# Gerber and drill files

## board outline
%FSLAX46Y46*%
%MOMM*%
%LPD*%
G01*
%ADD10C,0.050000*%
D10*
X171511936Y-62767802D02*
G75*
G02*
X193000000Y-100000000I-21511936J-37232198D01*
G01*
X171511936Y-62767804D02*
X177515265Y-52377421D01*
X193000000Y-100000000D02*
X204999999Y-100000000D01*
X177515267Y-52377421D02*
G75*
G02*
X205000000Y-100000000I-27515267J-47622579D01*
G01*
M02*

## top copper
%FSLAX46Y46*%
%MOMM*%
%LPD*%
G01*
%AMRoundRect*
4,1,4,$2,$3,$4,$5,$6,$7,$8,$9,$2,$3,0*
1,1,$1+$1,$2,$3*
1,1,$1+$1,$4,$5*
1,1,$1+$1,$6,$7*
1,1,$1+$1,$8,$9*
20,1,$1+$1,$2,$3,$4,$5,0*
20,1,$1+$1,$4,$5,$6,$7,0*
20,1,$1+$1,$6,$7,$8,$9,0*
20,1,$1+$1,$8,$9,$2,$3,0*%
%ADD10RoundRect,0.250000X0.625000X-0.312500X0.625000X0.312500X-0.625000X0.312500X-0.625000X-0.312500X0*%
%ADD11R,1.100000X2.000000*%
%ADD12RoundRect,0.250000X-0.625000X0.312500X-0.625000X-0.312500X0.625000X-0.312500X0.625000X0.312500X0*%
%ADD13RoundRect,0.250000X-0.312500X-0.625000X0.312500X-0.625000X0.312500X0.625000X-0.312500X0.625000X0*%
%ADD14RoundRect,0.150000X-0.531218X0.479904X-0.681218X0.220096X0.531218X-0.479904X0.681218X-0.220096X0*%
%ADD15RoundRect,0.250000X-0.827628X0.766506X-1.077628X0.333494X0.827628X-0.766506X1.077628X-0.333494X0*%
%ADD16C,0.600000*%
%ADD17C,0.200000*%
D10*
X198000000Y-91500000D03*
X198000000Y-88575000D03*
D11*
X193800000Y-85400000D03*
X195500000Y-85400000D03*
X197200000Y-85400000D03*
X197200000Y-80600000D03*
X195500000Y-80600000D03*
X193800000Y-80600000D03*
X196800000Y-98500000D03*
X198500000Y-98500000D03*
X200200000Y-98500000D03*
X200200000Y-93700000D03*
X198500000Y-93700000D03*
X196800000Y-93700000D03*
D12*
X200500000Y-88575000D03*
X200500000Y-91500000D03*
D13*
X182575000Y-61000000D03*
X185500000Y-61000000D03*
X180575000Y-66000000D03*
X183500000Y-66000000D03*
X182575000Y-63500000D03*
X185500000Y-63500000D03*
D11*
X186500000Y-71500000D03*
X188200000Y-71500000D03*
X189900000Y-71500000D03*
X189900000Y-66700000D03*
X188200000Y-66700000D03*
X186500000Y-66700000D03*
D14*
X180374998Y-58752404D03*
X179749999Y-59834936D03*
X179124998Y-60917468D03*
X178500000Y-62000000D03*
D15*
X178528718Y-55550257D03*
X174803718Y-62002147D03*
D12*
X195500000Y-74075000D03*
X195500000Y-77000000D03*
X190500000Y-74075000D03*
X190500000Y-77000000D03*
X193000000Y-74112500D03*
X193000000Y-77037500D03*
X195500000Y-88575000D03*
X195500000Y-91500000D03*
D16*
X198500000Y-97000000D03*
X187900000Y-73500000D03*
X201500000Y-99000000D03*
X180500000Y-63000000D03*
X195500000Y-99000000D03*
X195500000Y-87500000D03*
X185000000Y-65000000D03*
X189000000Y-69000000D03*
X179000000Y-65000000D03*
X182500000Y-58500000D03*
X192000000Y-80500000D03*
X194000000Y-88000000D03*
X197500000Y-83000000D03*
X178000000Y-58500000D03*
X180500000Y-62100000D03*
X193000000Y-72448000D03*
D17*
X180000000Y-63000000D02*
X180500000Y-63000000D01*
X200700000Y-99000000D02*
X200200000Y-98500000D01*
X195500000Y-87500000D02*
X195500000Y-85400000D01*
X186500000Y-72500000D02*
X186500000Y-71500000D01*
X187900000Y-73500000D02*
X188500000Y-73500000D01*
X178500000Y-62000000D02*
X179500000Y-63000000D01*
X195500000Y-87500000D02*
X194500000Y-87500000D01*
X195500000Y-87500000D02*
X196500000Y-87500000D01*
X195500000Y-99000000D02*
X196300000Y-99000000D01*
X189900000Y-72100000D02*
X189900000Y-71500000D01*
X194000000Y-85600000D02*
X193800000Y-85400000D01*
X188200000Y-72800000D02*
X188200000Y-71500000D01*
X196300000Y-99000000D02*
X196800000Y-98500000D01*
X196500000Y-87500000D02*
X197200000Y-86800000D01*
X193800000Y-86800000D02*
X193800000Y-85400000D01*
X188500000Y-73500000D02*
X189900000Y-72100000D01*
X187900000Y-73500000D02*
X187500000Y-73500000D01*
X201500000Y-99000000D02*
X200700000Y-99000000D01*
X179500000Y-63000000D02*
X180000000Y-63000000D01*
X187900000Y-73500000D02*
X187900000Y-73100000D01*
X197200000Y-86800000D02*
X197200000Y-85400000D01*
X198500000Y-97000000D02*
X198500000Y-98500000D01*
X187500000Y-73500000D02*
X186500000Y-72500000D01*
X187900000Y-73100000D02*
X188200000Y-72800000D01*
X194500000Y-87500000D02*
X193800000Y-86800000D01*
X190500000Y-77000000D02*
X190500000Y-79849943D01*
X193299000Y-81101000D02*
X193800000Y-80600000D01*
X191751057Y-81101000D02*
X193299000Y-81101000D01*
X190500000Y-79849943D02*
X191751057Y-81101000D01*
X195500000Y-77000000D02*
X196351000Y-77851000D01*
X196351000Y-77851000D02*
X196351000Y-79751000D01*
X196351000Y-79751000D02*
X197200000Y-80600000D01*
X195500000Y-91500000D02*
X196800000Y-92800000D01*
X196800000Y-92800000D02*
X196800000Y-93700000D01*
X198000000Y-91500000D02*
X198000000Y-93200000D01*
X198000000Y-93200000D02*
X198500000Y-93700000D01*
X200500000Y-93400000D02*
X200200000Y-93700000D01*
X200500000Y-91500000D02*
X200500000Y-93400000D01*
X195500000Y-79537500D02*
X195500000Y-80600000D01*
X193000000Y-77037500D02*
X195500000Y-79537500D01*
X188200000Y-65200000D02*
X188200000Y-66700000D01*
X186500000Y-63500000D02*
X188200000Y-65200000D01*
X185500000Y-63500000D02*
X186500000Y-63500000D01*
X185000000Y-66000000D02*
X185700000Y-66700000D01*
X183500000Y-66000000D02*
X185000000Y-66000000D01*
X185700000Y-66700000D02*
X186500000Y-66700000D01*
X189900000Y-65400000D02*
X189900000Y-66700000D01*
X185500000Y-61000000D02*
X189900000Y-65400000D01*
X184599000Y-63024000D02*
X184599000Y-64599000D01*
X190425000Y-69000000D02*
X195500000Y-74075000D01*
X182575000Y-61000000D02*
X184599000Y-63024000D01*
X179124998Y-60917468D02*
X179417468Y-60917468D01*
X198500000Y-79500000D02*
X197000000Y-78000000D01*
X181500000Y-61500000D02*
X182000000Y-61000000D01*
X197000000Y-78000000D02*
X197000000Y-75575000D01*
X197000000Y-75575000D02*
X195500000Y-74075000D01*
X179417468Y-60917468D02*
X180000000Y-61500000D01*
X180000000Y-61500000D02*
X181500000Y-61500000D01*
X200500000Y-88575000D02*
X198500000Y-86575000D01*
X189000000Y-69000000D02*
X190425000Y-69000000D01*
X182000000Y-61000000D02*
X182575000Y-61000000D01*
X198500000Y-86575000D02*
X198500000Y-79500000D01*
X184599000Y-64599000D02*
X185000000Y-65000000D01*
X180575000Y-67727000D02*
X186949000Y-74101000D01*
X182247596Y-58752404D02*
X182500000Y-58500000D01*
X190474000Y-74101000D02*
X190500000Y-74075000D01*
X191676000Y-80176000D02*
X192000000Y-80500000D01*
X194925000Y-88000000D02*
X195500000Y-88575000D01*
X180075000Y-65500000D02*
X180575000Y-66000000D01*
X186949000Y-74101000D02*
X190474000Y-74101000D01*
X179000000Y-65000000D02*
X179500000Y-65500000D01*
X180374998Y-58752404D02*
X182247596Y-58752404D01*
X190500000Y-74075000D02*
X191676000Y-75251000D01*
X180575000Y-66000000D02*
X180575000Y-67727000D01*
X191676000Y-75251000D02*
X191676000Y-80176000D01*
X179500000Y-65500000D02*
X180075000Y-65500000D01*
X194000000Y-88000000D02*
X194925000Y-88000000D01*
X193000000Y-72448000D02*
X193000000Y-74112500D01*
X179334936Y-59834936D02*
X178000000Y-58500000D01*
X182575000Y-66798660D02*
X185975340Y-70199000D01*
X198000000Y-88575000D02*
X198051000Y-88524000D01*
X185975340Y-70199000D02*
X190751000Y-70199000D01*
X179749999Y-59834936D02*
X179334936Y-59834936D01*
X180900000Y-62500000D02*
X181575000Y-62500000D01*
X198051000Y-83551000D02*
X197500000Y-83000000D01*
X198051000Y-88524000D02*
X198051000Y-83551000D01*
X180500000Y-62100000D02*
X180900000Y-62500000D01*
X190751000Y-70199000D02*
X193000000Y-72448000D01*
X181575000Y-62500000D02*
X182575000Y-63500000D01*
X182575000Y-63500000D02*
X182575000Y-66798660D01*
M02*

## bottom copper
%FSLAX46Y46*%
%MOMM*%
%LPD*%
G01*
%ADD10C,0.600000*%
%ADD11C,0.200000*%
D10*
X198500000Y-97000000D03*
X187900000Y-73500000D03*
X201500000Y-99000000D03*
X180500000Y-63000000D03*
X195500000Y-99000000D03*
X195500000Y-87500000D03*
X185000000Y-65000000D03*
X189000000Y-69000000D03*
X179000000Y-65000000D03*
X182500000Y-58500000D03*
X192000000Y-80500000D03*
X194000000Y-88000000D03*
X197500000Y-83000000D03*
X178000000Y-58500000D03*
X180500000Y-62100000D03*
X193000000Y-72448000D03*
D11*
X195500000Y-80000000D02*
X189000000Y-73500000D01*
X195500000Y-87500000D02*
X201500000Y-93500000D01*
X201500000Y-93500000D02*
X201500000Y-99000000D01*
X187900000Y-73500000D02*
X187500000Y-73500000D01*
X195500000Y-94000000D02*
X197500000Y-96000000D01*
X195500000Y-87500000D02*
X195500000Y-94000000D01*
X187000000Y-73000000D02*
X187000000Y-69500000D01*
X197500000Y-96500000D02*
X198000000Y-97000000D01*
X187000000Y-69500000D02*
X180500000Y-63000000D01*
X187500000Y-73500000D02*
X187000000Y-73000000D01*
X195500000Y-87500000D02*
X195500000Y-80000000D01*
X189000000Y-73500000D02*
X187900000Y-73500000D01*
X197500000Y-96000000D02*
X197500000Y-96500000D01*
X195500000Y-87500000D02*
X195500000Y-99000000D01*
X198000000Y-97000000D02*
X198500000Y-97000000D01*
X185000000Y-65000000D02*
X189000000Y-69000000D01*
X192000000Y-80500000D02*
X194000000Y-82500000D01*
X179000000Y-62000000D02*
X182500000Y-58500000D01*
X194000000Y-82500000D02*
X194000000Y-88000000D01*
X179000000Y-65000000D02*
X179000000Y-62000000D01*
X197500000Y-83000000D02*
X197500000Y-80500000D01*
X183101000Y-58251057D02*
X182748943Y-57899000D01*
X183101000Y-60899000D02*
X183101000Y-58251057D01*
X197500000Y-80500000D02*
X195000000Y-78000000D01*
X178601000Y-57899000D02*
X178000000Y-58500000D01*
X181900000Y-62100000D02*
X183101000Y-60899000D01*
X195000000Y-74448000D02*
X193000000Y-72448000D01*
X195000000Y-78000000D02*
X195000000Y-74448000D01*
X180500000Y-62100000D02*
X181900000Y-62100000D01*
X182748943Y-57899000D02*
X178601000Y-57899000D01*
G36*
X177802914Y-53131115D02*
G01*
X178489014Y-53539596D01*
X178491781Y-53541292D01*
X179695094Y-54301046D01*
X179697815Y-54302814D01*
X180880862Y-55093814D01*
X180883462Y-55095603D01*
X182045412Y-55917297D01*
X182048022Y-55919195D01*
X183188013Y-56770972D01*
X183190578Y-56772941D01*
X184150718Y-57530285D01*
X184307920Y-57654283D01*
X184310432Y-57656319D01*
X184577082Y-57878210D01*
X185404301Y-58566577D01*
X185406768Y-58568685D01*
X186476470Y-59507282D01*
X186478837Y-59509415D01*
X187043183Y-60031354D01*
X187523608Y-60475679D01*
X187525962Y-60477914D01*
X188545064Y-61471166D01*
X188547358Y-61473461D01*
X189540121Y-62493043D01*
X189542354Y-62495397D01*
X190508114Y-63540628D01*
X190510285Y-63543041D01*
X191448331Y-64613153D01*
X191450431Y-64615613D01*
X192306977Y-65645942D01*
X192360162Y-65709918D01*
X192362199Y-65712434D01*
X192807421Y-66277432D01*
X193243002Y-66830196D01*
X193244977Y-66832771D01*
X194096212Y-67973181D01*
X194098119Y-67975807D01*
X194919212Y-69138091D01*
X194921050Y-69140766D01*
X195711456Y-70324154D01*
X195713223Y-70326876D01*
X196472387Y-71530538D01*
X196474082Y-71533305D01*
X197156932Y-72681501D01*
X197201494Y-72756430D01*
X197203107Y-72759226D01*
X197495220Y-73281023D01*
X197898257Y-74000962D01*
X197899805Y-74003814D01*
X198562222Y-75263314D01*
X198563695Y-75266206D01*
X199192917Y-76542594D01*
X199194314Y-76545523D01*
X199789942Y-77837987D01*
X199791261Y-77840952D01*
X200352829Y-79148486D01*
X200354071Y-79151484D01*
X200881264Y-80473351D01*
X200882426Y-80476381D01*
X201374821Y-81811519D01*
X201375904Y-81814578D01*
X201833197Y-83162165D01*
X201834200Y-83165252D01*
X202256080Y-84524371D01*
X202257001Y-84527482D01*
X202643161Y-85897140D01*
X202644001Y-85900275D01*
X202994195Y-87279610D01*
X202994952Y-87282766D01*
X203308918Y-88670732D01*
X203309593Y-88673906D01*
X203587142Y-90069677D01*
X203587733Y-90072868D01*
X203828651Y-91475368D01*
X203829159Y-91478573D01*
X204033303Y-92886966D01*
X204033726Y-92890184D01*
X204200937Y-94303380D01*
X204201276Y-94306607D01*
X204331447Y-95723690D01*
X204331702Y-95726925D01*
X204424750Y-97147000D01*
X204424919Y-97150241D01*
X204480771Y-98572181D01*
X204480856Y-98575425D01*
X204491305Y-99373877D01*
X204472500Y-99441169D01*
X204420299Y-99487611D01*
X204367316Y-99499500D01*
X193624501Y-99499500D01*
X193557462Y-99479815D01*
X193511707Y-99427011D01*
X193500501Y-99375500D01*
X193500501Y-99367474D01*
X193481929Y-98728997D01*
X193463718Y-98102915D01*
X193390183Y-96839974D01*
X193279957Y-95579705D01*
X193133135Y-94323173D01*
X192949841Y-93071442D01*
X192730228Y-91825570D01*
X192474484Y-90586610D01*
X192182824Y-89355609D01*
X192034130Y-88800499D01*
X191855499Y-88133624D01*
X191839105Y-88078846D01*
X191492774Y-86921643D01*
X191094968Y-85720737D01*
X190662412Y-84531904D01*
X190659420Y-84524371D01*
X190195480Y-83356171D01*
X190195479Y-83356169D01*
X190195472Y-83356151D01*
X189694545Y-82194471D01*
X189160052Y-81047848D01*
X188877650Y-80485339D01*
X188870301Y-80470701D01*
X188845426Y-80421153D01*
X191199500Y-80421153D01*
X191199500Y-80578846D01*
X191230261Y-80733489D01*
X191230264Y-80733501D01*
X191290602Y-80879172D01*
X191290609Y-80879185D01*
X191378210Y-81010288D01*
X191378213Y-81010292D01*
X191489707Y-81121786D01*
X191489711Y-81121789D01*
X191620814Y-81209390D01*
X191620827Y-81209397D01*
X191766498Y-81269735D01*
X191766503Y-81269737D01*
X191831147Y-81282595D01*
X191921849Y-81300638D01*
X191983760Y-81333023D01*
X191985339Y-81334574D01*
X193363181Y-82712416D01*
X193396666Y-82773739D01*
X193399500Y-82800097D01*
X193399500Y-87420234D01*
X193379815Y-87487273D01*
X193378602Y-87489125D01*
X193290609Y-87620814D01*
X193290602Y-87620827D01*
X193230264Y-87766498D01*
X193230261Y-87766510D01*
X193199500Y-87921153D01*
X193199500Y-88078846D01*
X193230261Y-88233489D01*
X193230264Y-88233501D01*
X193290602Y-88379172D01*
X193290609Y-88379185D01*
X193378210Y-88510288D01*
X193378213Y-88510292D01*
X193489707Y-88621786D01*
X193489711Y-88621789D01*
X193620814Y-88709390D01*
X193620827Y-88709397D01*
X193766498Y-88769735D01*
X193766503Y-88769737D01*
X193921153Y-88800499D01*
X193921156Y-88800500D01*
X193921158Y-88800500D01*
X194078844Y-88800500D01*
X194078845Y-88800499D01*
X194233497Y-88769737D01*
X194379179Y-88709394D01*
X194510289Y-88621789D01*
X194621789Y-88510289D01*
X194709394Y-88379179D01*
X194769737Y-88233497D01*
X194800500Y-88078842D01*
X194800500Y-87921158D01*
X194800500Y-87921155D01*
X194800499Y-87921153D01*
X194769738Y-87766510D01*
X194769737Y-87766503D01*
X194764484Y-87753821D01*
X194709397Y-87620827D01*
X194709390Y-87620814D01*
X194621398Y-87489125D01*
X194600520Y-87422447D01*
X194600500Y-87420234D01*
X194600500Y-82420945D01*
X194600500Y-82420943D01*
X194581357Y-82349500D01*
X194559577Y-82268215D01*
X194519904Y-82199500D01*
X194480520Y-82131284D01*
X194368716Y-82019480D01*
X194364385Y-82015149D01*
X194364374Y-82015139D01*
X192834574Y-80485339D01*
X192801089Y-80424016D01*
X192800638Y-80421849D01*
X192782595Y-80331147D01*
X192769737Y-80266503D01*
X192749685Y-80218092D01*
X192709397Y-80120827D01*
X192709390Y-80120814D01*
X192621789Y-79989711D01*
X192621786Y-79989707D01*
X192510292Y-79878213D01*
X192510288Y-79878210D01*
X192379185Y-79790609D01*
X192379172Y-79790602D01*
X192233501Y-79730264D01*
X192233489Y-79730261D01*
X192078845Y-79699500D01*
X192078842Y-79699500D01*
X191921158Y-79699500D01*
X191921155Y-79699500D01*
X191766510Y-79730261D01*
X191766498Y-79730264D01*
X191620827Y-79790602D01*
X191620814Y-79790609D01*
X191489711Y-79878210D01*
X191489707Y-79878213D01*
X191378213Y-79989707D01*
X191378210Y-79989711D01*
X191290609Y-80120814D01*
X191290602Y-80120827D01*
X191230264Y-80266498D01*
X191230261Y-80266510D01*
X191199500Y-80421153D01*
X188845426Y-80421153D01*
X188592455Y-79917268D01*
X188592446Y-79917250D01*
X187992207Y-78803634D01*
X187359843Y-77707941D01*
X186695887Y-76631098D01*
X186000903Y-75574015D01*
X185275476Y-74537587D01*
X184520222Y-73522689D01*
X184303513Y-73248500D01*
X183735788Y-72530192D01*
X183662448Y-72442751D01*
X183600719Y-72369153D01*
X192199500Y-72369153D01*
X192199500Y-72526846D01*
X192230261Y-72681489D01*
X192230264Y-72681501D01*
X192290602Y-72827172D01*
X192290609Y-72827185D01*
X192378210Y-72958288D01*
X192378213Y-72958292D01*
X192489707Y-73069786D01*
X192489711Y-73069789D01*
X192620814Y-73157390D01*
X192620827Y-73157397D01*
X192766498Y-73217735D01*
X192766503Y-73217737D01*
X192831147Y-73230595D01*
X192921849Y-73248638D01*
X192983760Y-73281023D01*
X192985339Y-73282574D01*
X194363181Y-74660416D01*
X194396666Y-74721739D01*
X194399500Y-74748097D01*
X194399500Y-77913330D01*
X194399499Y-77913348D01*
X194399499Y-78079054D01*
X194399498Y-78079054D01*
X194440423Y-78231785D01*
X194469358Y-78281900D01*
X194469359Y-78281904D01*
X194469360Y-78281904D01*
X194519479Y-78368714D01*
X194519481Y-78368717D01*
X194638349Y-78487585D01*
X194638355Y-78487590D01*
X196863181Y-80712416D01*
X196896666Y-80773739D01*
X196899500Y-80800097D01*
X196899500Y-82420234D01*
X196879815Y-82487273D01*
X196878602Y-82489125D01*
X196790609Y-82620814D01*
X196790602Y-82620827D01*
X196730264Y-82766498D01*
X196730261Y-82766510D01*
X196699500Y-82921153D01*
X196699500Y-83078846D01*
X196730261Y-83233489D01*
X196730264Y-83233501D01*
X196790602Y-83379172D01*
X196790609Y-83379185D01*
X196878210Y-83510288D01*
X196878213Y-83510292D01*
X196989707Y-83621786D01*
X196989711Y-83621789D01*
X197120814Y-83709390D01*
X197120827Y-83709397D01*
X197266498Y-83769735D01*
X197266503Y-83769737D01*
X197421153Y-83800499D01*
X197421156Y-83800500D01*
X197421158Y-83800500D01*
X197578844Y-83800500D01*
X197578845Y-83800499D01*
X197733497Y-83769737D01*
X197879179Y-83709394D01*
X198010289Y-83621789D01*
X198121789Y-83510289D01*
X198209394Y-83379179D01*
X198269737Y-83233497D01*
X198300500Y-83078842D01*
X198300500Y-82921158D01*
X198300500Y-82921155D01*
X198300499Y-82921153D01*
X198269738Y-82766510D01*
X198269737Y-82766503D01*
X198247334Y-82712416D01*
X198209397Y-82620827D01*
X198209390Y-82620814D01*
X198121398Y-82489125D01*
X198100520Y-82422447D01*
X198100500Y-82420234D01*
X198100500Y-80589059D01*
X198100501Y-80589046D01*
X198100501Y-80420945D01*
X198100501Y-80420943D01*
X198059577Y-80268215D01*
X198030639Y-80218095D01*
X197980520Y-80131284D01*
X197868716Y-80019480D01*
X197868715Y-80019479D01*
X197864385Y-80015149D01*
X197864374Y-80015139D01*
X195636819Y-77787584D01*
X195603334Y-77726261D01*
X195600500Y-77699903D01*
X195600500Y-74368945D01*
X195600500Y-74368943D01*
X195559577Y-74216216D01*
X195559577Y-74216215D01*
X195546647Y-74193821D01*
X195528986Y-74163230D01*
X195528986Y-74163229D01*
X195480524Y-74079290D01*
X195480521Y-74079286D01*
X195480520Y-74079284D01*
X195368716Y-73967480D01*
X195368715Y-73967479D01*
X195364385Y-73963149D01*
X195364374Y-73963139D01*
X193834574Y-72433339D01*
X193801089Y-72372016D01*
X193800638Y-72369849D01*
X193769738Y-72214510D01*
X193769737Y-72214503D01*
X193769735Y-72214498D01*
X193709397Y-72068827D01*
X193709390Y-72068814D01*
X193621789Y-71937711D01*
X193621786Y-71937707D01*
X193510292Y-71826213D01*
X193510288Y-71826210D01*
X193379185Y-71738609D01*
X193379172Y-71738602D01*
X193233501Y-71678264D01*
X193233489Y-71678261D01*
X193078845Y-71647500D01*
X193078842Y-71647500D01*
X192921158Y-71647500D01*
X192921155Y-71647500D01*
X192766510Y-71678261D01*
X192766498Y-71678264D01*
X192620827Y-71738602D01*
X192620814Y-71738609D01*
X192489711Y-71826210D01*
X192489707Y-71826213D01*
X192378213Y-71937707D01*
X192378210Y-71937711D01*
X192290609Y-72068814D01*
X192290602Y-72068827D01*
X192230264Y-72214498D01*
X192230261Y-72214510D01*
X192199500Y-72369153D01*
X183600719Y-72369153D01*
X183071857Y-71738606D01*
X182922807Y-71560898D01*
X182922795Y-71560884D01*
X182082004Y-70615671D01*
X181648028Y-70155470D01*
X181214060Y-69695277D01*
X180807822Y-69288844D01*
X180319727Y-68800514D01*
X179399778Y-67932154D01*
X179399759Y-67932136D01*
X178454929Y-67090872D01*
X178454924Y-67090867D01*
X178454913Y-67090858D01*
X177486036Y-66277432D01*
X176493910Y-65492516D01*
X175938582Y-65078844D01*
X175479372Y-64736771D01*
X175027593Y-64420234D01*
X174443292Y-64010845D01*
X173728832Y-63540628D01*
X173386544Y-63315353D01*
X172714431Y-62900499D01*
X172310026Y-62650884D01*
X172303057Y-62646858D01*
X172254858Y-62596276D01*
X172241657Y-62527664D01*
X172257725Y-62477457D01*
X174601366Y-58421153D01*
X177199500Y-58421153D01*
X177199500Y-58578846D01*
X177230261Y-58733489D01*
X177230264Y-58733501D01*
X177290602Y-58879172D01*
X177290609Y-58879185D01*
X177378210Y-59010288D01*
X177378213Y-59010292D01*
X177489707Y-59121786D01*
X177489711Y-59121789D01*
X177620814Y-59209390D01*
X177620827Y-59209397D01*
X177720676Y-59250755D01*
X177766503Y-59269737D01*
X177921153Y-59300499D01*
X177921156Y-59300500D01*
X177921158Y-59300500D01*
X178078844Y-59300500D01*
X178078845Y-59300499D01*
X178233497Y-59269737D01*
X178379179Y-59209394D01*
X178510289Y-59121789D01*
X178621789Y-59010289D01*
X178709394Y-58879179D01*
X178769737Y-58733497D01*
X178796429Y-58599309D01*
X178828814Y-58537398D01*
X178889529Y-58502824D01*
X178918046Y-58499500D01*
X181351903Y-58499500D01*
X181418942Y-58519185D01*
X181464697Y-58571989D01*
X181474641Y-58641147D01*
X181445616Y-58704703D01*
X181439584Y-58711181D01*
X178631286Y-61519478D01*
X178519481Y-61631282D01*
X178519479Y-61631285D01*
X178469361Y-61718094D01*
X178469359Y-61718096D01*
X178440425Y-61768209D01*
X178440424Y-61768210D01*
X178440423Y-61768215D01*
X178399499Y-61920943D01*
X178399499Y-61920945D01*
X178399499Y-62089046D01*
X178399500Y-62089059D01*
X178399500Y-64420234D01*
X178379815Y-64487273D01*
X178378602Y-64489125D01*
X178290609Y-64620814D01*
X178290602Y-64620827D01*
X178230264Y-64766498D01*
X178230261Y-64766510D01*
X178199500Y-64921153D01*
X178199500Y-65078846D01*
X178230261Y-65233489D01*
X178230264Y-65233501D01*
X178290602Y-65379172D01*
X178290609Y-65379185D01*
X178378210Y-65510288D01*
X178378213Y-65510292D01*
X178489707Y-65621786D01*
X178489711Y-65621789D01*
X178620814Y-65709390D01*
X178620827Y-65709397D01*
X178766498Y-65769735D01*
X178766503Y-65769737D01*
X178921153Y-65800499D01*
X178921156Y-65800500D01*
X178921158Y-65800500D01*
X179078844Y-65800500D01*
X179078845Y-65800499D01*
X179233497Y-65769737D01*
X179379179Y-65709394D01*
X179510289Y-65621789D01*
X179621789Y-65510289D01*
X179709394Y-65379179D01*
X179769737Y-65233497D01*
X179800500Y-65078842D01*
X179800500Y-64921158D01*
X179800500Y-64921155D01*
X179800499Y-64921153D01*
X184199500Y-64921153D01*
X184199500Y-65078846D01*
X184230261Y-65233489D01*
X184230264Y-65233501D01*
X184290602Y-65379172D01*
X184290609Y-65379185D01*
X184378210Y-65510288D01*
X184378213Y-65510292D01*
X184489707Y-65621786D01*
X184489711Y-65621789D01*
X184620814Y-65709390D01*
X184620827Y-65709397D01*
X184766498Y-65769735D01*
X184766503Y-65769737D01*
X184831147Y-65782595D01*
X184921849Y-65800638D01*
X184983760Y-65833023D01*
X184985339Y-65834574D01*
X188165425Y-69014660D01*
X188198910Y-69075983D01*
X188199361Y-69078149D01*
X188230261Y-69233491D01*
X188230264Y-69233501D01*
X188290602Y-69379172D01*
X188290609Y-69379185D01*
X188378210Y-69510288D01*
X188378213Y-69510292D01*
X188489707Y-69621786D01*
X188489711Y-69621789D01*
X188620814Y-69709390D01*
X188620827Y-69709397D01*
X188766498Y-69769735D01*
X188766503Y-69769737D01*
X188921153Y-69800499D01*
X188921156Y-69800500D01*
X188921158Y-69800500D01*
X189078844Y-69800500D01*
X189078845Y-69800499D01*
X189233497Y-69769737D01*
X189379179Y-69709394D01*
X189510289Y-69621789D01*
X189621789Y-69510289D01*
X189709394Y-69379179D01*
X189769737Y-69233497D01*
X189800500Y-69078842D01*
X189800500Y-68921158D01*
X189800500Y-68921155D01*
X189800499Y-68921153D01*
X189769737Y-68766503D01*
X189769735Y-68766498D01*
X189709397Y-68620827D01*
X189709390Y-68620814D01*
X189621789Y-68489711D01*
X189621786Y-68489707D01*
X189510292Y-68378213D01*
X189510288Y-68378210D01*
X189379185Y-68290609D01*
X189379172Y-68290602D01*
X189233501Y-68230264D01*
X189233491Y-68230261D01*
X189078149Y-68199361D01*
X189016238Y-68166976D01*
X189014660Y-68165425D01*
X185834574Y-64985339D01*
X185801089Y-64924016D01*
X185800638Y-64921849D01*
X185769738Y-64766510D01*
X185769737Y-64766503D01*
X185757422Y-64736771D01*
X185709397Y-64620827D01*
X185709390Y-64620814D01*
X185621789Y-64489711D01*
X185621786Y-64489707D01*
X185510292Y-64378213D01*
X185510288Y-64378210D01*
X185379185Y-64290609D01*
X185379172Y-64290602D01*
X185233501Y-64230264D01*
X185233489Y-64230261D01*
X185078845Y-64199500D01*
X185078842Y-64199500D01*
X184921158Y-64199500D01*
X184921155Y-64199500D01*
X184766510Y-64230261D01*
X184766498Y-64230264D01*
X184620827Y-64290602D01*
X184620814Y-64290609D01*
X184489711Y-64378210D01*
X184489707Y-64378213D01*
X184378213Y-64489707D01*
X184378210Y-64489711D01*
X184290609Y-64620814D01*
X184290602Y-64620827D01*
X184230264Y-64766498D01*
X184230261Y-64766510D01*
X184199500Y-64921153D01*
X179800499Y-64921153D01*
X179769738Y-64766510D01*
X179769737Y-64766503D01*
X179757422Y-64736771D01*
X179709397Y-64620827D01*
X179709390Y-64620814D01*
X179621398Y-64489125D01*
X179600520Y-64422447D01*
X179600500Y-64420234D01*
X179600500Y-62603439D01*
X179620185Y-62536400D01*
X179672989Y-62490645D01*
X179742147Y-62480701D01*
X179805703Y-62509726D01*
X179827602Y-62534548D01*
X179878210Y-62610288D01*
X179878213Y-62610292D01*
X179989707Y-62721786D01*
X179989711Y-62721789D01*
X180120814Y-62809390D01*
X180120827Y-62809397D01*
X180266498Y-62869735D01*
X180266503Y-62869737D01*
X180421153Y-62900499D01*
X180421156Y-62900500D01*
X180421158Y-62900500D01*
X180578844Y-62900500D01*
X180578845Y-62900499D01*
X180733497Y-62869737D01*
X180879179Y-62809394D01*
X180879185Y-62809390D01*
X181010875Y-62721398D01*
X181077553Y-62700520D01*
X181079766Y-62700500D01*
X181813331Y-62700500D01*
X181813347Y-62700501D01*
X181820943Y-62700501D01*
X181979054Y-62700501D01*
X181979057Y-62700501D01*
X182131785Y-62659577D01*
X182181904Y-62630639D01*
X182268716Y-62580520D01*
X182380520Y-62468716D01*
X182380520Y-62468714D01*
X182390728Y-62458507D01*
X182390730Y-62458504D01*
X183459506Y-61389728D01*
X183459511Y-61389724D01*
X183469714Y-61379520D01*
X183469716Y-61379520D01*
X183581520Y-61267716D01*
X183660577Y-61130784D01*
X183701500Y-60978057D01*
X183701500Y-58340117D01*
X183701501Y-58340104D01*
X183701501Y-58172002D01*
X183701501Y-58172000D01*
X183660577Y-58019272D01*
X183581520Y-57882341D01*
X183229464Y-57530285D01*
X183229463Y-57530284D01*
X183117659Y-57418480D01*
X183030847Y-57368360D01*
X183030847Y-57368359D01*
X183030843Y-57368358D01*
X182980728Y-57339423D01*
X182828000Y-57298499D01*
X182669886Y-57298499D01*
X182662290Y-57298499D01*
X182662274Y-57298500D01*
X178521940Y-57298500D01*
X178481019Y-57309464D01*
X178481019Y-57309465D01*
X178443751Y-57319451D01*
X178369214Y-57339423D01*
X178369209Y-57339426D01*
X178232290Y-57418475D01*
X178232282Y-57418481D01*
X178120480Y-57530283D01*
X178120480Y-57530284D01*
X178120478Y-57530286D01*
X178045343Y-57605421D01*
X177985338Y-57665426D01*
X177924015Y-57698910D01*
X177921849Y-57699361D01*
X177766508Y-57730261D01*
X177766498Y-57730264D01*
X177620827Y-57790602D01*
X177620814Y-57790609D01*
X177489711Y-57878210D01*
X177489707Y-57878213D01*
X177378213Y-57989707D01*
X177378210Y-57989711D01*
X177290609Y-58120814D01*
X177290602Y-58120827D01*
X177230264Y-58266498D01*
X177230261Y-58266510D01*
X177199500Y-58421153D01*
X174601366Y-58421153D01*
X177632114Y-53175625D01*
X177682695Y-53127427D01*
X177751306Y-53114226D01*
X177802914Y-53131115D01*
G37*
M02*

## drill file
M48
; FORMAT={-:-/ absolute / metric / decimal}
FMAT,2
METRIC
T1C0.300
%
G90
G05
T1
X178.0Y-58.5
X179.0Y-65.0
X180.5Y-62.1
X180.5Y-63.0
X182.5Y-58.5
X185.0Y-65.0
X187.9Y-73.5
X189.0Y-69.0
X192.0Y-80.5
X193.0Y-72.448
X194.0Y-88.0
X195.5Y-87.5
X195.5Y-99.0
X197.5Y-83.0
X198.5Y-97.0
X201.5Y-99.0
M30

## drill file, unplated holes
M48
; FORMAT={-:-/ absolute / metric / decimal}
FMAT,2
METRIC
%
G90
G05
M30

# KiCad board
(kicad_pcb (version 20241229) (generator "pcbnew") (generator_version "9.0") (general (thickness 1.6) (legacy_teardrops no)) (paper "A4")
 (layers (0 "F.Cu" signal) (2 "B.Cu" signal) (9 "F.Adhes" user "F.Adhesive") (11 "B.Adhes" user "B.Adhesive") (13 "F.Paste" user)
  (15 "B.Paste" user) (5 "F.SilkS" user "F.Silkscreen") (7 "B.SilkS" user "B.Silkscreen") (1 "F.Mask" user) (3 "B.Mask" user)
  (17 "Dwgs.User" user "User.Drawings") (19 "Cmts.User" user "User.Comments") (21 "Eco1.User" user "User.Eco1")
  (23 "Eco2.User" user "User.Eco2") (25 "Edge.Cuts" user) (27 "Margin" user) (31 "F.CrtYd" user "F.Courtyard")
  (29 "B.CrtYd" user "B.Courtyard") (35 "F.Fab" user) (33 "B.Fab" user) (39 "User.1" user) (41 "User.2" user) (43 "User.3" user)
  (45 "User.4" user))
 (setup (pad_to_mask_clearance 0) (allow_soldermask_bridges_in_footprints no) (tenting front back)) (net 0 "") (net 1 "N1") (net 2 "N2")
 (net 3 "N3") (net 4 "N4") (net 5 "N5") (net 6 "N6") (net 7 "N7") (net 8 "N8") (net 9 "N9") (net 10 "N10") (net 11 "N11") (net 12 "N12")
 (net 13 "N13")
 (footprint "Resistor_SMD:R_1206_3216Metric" (layer "F.Cu") (at 198 90.0375 90)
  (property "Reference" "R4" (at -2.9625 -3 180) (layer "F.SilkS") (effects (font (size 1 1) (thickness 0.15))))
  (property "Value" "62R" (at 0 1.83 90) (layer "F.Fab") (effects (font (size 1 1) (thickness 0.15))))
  (pad "1" smd roundrect (at -1.4625 0 90) (size 1.125 1.75) (layers "F.Cu" "F.Mask" "F.Paste") (roundrect_rratio 0.222222) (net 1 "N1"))
  (pad "2" smd roundrect (at 1.4625 0 90) (size 1.125 1.75) (layers "F.Cu" "F.Mask" "F.Paste") (roundrect_rratio 0.222222) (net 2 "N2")))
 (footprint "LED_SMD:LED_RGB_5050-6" (layer "F.Cu") (at 195.5 83 90)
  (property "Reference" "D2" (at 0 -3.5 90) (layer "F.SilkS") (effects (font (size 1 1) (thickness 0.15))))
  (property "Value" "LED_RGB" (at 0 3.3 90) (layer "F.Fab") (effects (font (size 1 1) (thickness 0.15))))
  (pad "1" smd rect (at -2.4 -1.7 180) (size 1.1 2) (layers "F.Cu" "F.Mask" "F.Paste") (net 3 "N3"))
  (pad "2" smd rect (at -2.4 0 180) (size 1.1 2) (layers "F.Cu" "F.Mask" "F.Paste") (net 3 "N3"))
  (pad "3" smd rect (at -2.4 1.7 180) (size 1.1 2) (layers "F.Cu" "F.Mask" "F.Paste") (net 3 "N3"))
  (pad "4" smd rect (at 2.4 1.7 180) (size 1.1 2) (layers "F.Cu" "F.Mask" "F.Paste") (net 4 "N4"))
  (pad "5" smd rect (at 2.4 0 180) (size 1.1 2) (layers "F.Cu" "F.Mask" "F.Paste") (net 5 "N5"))
  (pad "6" smd rect (at 2.4 -1.7 180) (size 1.1 2) (layers "F.Cu" "F.Mask" "F.Paste") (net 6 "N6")))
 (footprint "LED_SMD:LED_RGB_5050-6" (layer "F.Cu") (at 198.5 96.1 90)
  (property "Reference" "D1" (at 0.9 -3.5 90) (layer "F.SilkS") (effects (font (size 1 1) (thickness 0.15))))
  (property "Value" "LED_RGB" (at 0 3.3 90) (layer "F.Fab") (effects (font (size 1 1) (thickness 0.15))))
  (pad "1" smd rect (at -2.4 -1.7 180) (size 1.1 2) (layers "F.Cu" "F.Mask" "F.Paste") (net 3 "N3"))
  (pad "2" smd rect (at -2.4 0 180) (size 1.1 2) (layers "F.Cu" "F.Mask" "F.Paste") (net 3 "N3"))
  (pad "3" smd rect (at -2.4 1.7 180) (size 1.1 2) (layers "F.Cu" "F.Mask" "F.Paste") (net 3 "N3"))
  (pad "4" smd rect (at 2.4 1.7 180) (size 1.1 2) (layers "F.Cu" "F.Mask" "F.Paste") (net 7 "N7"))
  (pad "5" smd rect (at 2.4 0 180) (size 1.1 2) (layers "F.Cu" "F.Mask" "F.Paste") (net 1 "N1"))
  (pad "6" smd rect (at 2.4 -1.7 180) (size 1.1 2) (layers "F.Cu" "F.Mask" "F.Paste") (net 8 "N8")))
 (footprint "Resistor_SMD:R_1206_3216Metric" (layer "F.Cu") (at 200.5 90.0375 -90)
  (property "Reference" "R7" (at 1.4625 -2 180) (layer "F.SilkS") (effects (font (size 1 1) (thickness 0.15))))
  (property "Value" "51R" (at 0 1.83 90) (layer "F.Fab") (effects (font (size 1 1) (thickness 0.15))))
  (pad "1" smd roundrect (at -1.4625 0 270) (size 1.125 1.75) (layers "F.Cu" "F.Mask" "F.Paste") (roundrect_rratio 0.222222) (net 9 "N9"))
  (pad "2" smd roundrect (at 1.4625 0 270) (size 1.125 1.75) (layers "F.Cu" "F.Mask" "F.Paste") (roundrect_rratio 0.222222) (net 7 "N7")))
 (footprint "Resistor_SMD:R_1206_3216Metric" (layer "F.Cu") (at 184.0375 61)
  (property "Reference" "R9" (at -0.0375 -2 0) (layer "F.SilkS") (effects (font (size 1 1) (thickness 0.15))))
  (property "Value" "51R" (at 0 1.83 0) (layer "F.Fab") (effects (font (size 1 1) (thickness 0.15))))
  (pad "1" smd roundrect (at -1.4625 0) (size 1.125 1.75) (layers "F.Cu" "F.Mask" "F.Paste") (roundrect_rratio 0.222222) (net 9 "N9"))
  (pad "2" smd roundrect (at 1.4625 0) (size 1.125 1.75) (layers "F.Cu" "F.Mask" "F.Paste") (roundrect_rratio 0.222222) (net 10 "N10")))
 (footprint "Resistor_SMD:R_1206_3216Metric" (layer "F.Cu") (at 182.0375 66)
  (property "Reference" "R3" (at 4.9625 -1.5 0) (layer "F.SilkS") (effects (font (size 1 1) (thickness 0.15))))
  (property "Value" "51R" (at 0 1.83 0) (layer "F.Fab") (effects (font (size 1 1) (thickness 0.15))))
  (pad "1" smd roundrect (at -1.4625 0) (size 1.125 1.75) (layers "F.Cu" "F.Mask" "F.Paste") (roundrect_rratio 0.222222) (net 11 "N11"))
  (pad "2" smd roundrect (at 1.4625 0) (size 1.125 1.75) (layers "F.Cu" "F.Mask" "F.Paste") (roundrect_rratio 0.222222) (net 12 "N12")))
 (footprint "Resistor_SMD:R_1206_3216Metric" (layer "F.Cu") (at 184.0375 63.5)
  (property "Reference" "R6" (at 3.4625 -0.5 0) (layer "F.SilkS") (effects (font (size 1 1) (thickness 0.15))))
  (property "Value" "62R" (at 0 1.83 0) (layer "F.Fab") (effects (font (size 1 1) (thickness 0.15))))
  (pad "1" smd roundrect (at -1.4625 0) (size 1.125 1.75) (layers "F.Cu" "F.Mask" "F.Paste") (roundrect_rratio 0.222222) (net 2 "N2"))
  (pad "2" smd roundrect (at 1.4625 0) (size 1.125 1.75) (layers "F.Cu" "F.Mask" "F.Paste") (roundrect_rratio 0.222222) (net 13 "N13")))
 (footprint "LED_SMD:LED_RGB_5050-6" (layer "F.Cu") (at 188.2 69.1 90)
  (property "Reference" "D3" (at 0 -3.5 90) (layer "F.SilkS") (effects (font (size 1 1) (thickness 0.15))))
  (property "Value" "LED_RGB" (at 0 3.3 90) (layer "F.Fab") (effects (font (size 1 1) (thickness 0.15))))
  (pad "1" smd rect (at -2.4 -1.7 180) (size 1.1 2) (layers "F.Cu" "F.Mask" "F.Paste") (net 3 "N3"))
  (pad "2" smd rect (at -2.4 0 180) (size 1.1 2) (layers "F.Cu" "F.Mask" "F.Paste") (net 3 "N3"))
  (pad "3" smd rect (at -2.4 1.7 180) (size 1.1 2) (layers "F.Cu" "F.Mask" "F.Paste") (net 3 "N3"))
  (pad "4" smd rect (at 2.4 1.7 180) (size 1.1 2) (layers "F.Cu" "F.Mask" "F.Paste") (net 10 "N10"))
  (pad "5" smd rect (at 2.4 0 180) (size 1.1 2) (layers "F.Cu" "F.Mask" "F.Paste") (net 13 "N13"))
  (pad "6" smd rect (at 2.4 -1.7 180) (size 1.1 2) (layers "F.Cu" "F.Mask" "F.Paste") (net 12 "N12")))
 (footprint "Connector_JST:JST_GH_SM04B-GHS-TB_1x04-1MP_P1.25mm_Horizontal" (layer "F.Cu") (at 177.835352 59.451202 -120)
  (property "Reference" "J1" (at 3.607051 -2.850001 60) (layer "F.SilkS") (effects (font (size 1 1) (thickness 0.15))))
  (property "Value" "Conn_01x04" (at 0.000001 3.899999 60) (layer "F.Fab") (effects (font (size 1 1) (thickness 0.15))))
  (pad "1" smd roundrect (at -1.875 -1.849999 240) (size 0.6 1.7) (layers "F.Cu" "F.Mask" "F.Paste") (roundrect_rratio 0.25) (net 11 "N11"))
  (pad "2" smd roundrect (at -0.625 -1.85 240) (size 0.6 1.7) (layers "F.Cu" "F.Mask" "F.Paste") (roundrect_rratio 0.25) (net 2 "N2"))
  (pad "3" smd roundrect (at 0.625001 -1.849999 240) (size 0.6 1.7) (layers "F.Cu" "F.Mask" "F.Paste") (roundrect_rratio 0.25) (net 9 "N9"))
  (pad "4" smd roundrect (at 1.875 -1.850001 240) (size 0.6 1.7) (layers "F.Cu" "F.Mask" "F.Paste") (roundrect_rratio 0.25) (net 3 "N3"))
  (pad "MP" smd roundrect (at -3.725 1.35 240) (size 1 2.7) (layers "F.Cu" "F.Mask" "F.Paste") (roundrect_rratio 0.25))
  (pad "MP" smd roundrect (at 3.725 1.35 240) (size 1 2.7) (layers "F.Cu" "F.Mask" "F.Paste") (roundrect_rratio 0.25)))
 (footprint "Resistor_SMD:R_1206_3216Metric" (layer "F.Cu") (at 195.5 75.5375 -90)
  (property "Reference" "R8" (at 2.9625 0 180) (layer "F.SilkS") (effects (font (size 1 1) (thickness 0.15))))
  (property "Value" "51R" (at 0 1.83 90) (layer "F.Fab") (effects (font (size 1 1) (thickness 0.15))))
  (pad "1" smd roundrect (at -1.4625 0 270) (size 1.125 1.75) (layers "F.Cu" "F.Mask" "F.Paste") (roundrect_rratio 0.222222) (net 9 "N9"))
  (pad "2" smd roundrect (at 1.4625 0 270) (size 1.125 1.75) (layers "F.Cu" "F.Mask" "F.Paste") (roundrect_rratio 0.222222) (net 4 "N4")))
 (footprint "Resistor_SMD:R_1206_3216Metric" (layer "F.Cu") (at 190.5 75.5375 -90)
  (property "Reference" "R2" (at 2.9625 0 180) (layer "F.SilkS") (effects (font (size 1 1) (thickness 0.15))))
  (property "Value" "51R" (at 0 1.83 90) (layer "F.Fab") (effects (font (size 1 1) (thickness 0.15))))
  (pad "1" smd roundrect (at -1.4625 0 270) (size 1.125 1.75) (layers "F.Cu" "F.Mask" "F.Paste") (roundrect_rratio 0.222222) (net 11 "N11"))
  (pad "2" smd roundrect (at 1.4625 0 270) (size 1.125 1.75) (layers "F.Cu" "F.Mask" "F.Paste") (roundrect_rratio 0.222222) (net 6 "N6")))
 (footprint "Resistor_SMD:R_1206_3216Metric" (layer "F.Cu") (at 193 75.575 -90)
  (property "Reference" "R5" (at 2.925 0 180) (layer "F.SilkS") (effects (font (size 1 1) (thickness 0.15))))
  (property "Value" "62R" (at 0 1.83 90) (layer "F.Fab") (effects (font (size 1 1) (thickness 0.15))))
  (pad "1" smd roundrect (at -1.4625 0 270) (size 1.125 1.75) (layers "F.Cu" "F.Mask" "F.Paste") (roundrect_rratio 0.222222) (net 2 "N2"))
  (pad "2" smd roundrect (at 1.4625 0 270) (size 1.125 1.75) (layers "F.Cu" "F.Mask" "F.Paste") (roundrect_rratio 0.222222) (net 5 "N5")))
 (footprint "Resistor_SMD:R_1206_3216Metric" (layer "F.Cu") (at 195.5 90.0375 -90)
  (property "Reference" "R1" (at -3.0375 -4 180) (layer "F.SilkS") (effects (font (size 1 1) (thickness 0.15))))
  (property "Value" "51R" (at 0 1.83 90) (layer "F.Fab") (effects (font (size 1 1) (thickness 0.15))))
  (pad "1" smd roundrect (at -1.4625 0 270) (size 1.125 1.75) (layers "F.Cu" "F.Mask" "F.Paste") (roundrect_rratio 0.222222) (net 11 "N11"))
  (pad "2" smd roundrect (at 1.4625 0 270) (size 1.125 1.75) (layers "F.Cu" "F.Mask" "F.Paste") (roundrect_rratio 0.222222) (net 8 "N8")))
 (gr_arc (start 171.511936 62.767802) (mid 187.242537 78.505969) (end 193 100) (stroke (width 0.05) (type default)) (layer "Edge.Cuts"))
 (gr_line (start 171.511936 62.767804) (end 177.515265 52.377421) (stroke (width 0.05) (type default)) (layer "Edge.Cuts"))
 (gr_line (start 193 100) (end 204.999999 100) (stroke (width 0.05) (type default)) (layer "Edge.Cuts"))
 (gr_arc (start 177.515267 52.377421) (mid 197.635804 72.507635) (end 205 100) (stroke (width 0.05) (type default)) (layer "Edge.Cuts"))
 (segment (start 180 63) (end 180.5 63) (width 0.2) (layer "F.Cu") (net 3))
 (segment (start 200.7 99) (end 200.2 98.5) (width 0.2) (layer "F.Cu") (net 3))
 (segment (start 195.5 87.5) (end 195.5 85.4) (width 0.2) (layer "F.Cu") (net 3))
 (segment (start 186.5 72.5) (end 186.5 71.5) (width 0.2) (layer "F.Cu") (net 3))
 (segment (start 187.9 73.5) (end 188.5 73.5) (width 0.2) (layer "F.Cu") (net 3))
 (segment (start 178.5 62) (end 179.5 63) (width 0.2) (layer "F.Cu") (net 3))
 (segment (start 195.5 87.5) (end 194.5 87.5) (width 0.2) (layer "F.Cu") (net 3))
 (segment (start 195.5 87.5) (end 196.5 87.5) (width 0.2) (layer "F.Cu") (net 3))
 (segment (start 195.5 99) (end 196.3 99) (width 0.2) (layer "F.Cu") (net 3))
 (segment (start 189.9 72.1) (end 189.9 71.5) (width 0.2) (layer "F.Cu") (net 3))
 (segment (start 194 85.6) (end 193.8 85.4) (width 0.2) (layer "F.Cu") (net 3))
 (segment (start 188.2 72.8) (end 188.2 71.5) (width 0.2) (layer "F.Cu") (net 3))
 (segment (start 196.3 99) (end 196.8 98.5) (width 0.2) (layer "F.Cu") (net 3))
 (segment (start 196.5 87.5) (end 197.2 86.8) (width 0.2) (layer "F.Cu") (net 3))
 (segment (start 193.8 86.8) (end 193.8 85.4) (width 0.2) (layer "F.Cu") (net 3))
 (segment (start 188.5 73.5) (end 189.9 72.1) (width 0.2) (layer "F.Cu") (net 3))
 (segment (start 187.9 73.5) (end 187.5 73.5) (width 0.2) (layer "F.Cu") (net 3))
 (segment (start 201.5 99) (end 200.7 99) (width 0.2) (layer "F.Cu") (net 3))
 (segment (start 179.5 63) (end 180 63) (width 0.2) (layer "F.Cu") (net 3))
 (segment (start 187.9 73.5) (end 187.9 73.1) (width 0.2) (layer "F.Cu") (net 3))
 (segment (start 197.2 86.8) (end 197.2 85.4) (width 0.2) (layer "F.Cu") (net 3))
 (segment (start 198.5 97) (end 198.5 98.5) (width 0.2) (layer "F.Cu") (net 3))
 (segment (start 187.5 73.5) (end 186.5 72.5) (width 0.2) (layer "F.Cu") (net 3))
 (segment (start 187.9 73.1) (end 188.2 72.8) (width 0.2) (layer "F.Cu") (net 3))
 (segment (start 194.5 87.5) (end 193.8 86.8) (width 0.2) (layer "F.Cu") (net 3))
 (via (at 198.5 97) (size 0.6) (drill 0.3) (layers "F.Cu" "B.Cu") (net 3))
 (via (at 187.9 73.5) (size 0.6) (drill 0.3) (layers "F.Cu" "B.Cu") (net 3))
 (via (at 201.5 99) (size 0.6) (drill 0.3) (layers "F.Cu" "B.Cu") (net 3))
 (via (at 180.5 63) (size 0.6) (drill 0.3) (layers "F.Cu" "B.Cu") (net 3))
 (via (at 195.5 99) (size 0.6) (drill 0.3) (layers "F.Cu" "B.Cu") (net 3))
 (via (at 195.5 87.5) (size 0.6) (drill 0.3) (layers "F.Cu" "B.Cu") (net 3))
 (segment (start 195.5 80) (end 189 73.5) (width 0.2) (layer "B.Cu") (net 3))
 (segment (start 195.5 87.5) (end 201.5 93.5) (width 0.2) (layer "B.Cu") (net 3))
 (segment (start 201.5 93.5) (end 201.5 99) (width 0.2) (layer "B.Cu") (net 3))
 (segment (start 187.9 73.5) (end 187.5 73.5) (width 0.2) (layer "B.Cu") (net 3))
 (segment (start 195.5 94) (end 197.5 96) (width 0.2) (layer "B.Cu") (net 3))
 (segment (start 195.5 87.5) (end 195.5 94) (width 0.2) (layer "B.Cu") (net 3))
 (segment (start 187 73) (end 187 69.5) (width 0.2) (layer "B.Cu") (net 3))
 (segment (start 197.5 96.5) (end 198 97) (width 0.2) (layer "B.Cu") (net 3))
 (segment (start 187 69.5) (end 180.5 63) (width 0.2) (layer "B.Cu") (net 3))
 (segment (start 187.5 73.5) (end 187 73) (width 0.2) (layer "B.Cu") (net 3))
 (segment (start 195.5 87.5) (end 195.5 80) (width 0.2) (layer "B.Cu") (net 3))
 (segment (start 189 73.5) (end 187.9 73.5) (width 0.2) (layer "B.Cu") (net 3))
 (segment (start 197.5 96) (end 197.5 96.5) (width 0.2) (layer "B.Cu") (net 3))
 (segment (start 195.5 87.5) (end 195.5 99) (width 0.2) (layer "B.Cu") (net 3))
 (segment (start 198 97) (end 198.5 97) (width 0.2) (layer "B.Cu") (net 3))
 (segment (start 190.5 77) (end 190.5 79.849943) (width 0.2) (layer "F.Cu") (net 6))
 (segment (start 193.299 81.101) (end 193.8 80.6) (width 0.2) (layer "F.Cu") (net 6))
 (segment (start 191.751057 81.101) (end 193.299 81.101) (width 0.2) (layer "F.Cu") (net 6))
 (segment (start 190.5 79.849943) (end 191.751057 81.101) (width 0.2) (layer "F.Cu") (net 6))
 (segment (start 195.5 77) (end 196.351 77.851) (width 0.2) (layer "F.Cu") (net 4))
 (segment (start 196.351 77.851) (end 196.351 79.751) (width 0.2) (layer "F.Cu") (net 4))
 (segment (start 196.351 79.751) (end 197.2 80.6) (width 0.2) (layer "F.Cu") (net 4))
 (segment (start 195.5 91.5) (end 196.8 92.8) (width 0.2) (layer "F.Cu") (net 8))
 (segment (start 196.8 92.8) (end 196.8 93.7) (width 0.2) (layer "F.Cu") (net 8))
 (segment (start 198 91.5) (end 198 93.2) (width 0.2) (layer "F.Cu") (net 1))
 (segment (start 198 93.2) (end 198.5 93.7) (width 0.2) (layer "F.Cu") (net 1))
 (segment (start 200.5 93.4) (end 200.2 93.7) (width 0.2) (layer "F.Cu") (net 7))
 (segment (start 200.5 91.5) (end 200.5 93.4) (width 0.2) (layer "F.Cu") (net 7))
 (segment (start 195.5 79.5375) (end 195.5 80.6) (width 0.2) (layer "F.Cu") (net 5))
 (segment (start 193 77.0375) (end 195.5 79.5375) (width 0.2) (layer "F.Cu") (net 5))
 (segment (start 188.2 65.2) (end 188.2 66.7) (width 0.2) (layer "F.Cu") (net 13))
 (segment (start 186.5 63.5) (end 188.2 65.2) (width 0.2) (layer "F.Cu") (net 13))
 (segment (start 185.5 63.5) (end 186.5 63.5) (width 0.2) (layer "F.Cu") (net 13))
 (segment (start 185 66) (end 185.7 66.7) (width 0.2) (layer "F.Cu") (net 12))
 (segment (start 183.5 66) (end 185 66) (width 0.2) (layer "F.Cu") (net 12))
 (segment (start 185.7 66.7) (end 186.5 66.7) (width 0.2) (layer "F.Cu") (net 12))
 (segment (start 189.9 65.4) (end 189.9 66.7) (width 0.2) (layer "F.Cu") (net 10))
 (segment (start 185.5 61) (end 189.9 65.4) (width 0.2) (layer "F.Cu") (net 10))
 (segment (start 184.599 63.024) (end 184.599 64.599) (width 0.2) (layer "F.Cu") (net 9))
 (segment (start 190.425 69) (end 195.5 74.075) (width 0.2) (layer "F.Cu") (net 9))
 (segment (start 182.575 61) (end 184.599 63.024) (width 0.2) (layer "F.Cu") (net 9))
 (segment (start 179.124998 60.917468) (end 179.417468 60.917468) (width 0.2) (layer "F.Cu") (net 9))
 (segment (start 198.5 79.5) (end 197 78) (width 0.2) (layer "F.Cu") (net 9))
 (segment (start 181.5 61.5) (end 182 61) (width 0.2) (layer "F.Cu") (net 9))
 (segment (start 197 78) (end 197 75.575) (width 0.2) (layer "F.Cu") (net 9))
 (segment (start 197 75.575) (end 195.5 74.075) (width 0.2) (layer "F.Cu") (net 9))
 (segment (start 179.417468 60.917468) (end 180 61.5) (width 0.2) (layer "F.Cu") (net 9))
 (segment (start 180 61.5) (end 181.5 61.5) (width 0.2) (layer "F.Cu") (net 9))
 (segment (start 200.5 88.575) (end 198.5 86.575) (width 0.2) (layer "F.Cu") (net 9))
 (segment (start 189 69) (end 190.425 69) (width 0.2) (layer "F.Cu") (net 9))
 (segment (start 182 61) (end 182.575 61) (width 0.2) (layer "F.Cu") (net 9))
 (segment (start 198.5 86.575) (end 198.5 79.5) (width 0.2) (layer "F.Cu") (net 9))
 (segment (start 184.599 64.599) (end 185 65) (width 0.2) (layer "F.Cu") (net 9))
 (via (at 185 65) (size 0.6) (drill 0.3) (layers "F.Cu" "B.Cu") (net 9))
 (via (at 189 69) (size 0.6) (drill 0.3) (layers "F.Cu" "B.Cu") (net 9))
 (segment (start 185 65) (end 189 69) (width 0.2) (layer "B.Cu") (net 9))
 (segment (start 180.575 67.727) (end 186.949 74.101) (width 0.2) (layer "F.Cu") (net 11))
 (segment (start 182.247596 58.752404) (end 182.5 58.5) (width 0.2) (layer "F.Cu") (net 11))
 (segment (start 190.474 74.101) (end 190.5 74.075) (width 0.2) (layer "F.Cu") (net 11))
 (segment (start 191.676 80.176) (end 192 80.5) (width 0.2) (layer "F.Cu") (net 11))
 (segment (start 194.925 88) (end 195.5 88.575) (width 0.2) (layer "F.Cu") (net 11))
 (segment (start 180.075 65.5) (end 180.575 66) (width 0.2) (layer "F.Cu") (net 11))
 (segment (start 186.949 74.101) (end 190.474 74.101) (width 0.2) (layer "F.Cu") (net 11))
 (segment (start 179 65) (end 179.5 65.5) (width 0.2) (layer "F.Cu") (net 11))
 (segment (start 180.374998 58.752404) (end 182.247596 58.752404) (width 0.2) (layer "F.Cu") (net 11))
 (segment (start 190.5 74.075) (end 191.676 75.251) (width 0.2) (layer "F.Cu") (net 11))
 (segment (start 180.575 66) (end 180.575 67.727) (width 0.2) (layer "F.Cu") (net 11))
 (segment (start 191.676 75.251) (end 191.676 80.176) (width 0.2) (layer "F.Cu") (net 11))
 (segment (start 179.5 65.5) (end 180.075 65.5) (width 0.2) (layer "F.Cu") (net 11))
 (segment (start 194 88) (end 194.925 88) (width 0.2) (layer "F.Cu") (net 11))
 (via (at 179 65) (size 0.6) (drill 0.3) (layers "F.Cu" "B.Cu") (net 11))
 (via (at 182.5 58.5) (size 0.6) (drill 0.3) (layers "F.Cu" "B.Cu") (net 11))
 (via (at 192 80.5) (size 0.6) (drill 0.3) (layers "F.Cu" "B.Cu") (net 11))
 (via (at 194 88) (size 0.6) (drill 0.3) (layers "F.Cu" "B.Cu") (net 11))
 (segment (start 192 80.5) (end 194 82.5) (width 0.2) (layer "B.Cu") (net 11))
 (segment (start 179 62) (end 182.5 58.5) (width 0.2) (layer "B.Cu") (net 11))
 (segment (start 194 82.5) (end 194 88) (width 0.2) (layer "B.Cu") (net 11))
 (segment (start 179 65) (end 179 62) (width 0.2) (layer "B.Cu") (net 11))
 (segment (start 193 72.448) (end 193 74.1125) (width 0.2) (layer "F.Cu") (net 2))
 (segment (start 179.334936 59.834936) (end 178 58.5) (width 0.2) (layer "F.Cu") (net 2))
 (segment (start 182.575 66.79866) (end 185.97534 70.199) (width 0.2) (layer "F.Cu") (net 2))
 (segment (start 198 88.575) (end 198.051 88.524) (width 0.2) (layer "F.Cu") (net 2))
 (segment (start 185.97534 70.199) (end 190.751 70.199) (width 0.2) (layer "F.Cu") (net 2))
 (segment (start 179.749999 59.834936) (end 179.334936 59.834936) (width 0.2) (layer "F.Cu") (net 2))
 (segment (start 180.9 62.5) (end 181.575 62.5) (width 0.2) (layer "F.Cu") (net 2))
 (segment (start 198.051 83.551) (end 197.5 83) (width 0.2) (layer "F.Cu") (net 2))
 (segment (start 198.051 88.524) (end 198.051 83.551) (width 0.2) (layer "F.Cu") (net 2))
 (segment (start 180.5 62.1) (end 180.9 62.5) (width 0.2) (layer "F.Cu") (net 2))
 (segment (start 190.751 70.199) (end 193 72.448) (width 0.2) (layer "F.Cu") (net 2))
 (segment (start 181.575 62.5) (end 182.575 63.5) (width 0.2) (layer "F.Cu") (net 2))
 (segment (start 182.575 63.5) (end 182.575 66.79866) (width 0.2) (layer "F.Cu") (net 2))
 (via (at 197.5 83) (size 0.6) (drill 0.3) (layers "F.Cu" "B.Cu") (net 2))
 (via (at 178 58.5) (size 0.6) (drill 0.3) (layers "F.Cu" "B.Cu") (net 2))
 (via (at 180.5 62.1) (size 0.6) (drill 0.3) (layers "F.Cu" "B.Cu") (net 2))
 (via (at 193 72.448) (size 0.6) (drill 0.3) (layers "F.Cu" "B.Cu") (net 2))
 (segment (start 197.5 83) (end 197.5 80.5) (width 0.2) (layer "B.Cu") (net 2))
 (segment (start 183.101 58.251057) (end 182.748943 57.899) (width 0.2) (layer "B.Cu") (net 2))
 (segment (start 183.101 60.899) (end 183.101 58.251057) (width 0.2) (layer "B.Cu") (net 2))
 (segment (start 197.5 80.5) (end 195 78) (width 0.2) (layer "B.Cu") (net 2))
 (segment (start 178.601 57.899) (end 178 58.5) (width 0.2) (layer "B.Cu") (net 2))
 (segment (start 181.9 62.1) (end 183.101 60.899) (width 0.2) (layer "B.Cu") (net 2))
 (segment (start 195 74.448) (end 193 72.448) (width 0.2) (layer "B.Cu") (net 2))
 (segment (start 195 78) (end 195 74.448) (width 0.2) (layer "B.Cu") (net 2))
 (segment (start 180.5 62.1) (end 181.9 62.1) (width 0.2) (layer "B.Cu") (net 2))
 (segment (start 182.748943 57.899) (end 178.601 57.899) (width 0.2) (layer "B.Cu") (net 2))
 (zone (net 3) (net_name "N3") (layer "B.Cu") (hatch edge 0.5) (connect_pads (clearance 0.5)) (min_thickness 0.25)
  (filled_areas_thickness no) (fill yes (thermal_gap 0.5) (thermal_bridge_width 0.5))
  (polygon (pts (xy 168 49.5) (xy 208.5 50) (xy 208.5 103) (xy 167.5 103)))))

